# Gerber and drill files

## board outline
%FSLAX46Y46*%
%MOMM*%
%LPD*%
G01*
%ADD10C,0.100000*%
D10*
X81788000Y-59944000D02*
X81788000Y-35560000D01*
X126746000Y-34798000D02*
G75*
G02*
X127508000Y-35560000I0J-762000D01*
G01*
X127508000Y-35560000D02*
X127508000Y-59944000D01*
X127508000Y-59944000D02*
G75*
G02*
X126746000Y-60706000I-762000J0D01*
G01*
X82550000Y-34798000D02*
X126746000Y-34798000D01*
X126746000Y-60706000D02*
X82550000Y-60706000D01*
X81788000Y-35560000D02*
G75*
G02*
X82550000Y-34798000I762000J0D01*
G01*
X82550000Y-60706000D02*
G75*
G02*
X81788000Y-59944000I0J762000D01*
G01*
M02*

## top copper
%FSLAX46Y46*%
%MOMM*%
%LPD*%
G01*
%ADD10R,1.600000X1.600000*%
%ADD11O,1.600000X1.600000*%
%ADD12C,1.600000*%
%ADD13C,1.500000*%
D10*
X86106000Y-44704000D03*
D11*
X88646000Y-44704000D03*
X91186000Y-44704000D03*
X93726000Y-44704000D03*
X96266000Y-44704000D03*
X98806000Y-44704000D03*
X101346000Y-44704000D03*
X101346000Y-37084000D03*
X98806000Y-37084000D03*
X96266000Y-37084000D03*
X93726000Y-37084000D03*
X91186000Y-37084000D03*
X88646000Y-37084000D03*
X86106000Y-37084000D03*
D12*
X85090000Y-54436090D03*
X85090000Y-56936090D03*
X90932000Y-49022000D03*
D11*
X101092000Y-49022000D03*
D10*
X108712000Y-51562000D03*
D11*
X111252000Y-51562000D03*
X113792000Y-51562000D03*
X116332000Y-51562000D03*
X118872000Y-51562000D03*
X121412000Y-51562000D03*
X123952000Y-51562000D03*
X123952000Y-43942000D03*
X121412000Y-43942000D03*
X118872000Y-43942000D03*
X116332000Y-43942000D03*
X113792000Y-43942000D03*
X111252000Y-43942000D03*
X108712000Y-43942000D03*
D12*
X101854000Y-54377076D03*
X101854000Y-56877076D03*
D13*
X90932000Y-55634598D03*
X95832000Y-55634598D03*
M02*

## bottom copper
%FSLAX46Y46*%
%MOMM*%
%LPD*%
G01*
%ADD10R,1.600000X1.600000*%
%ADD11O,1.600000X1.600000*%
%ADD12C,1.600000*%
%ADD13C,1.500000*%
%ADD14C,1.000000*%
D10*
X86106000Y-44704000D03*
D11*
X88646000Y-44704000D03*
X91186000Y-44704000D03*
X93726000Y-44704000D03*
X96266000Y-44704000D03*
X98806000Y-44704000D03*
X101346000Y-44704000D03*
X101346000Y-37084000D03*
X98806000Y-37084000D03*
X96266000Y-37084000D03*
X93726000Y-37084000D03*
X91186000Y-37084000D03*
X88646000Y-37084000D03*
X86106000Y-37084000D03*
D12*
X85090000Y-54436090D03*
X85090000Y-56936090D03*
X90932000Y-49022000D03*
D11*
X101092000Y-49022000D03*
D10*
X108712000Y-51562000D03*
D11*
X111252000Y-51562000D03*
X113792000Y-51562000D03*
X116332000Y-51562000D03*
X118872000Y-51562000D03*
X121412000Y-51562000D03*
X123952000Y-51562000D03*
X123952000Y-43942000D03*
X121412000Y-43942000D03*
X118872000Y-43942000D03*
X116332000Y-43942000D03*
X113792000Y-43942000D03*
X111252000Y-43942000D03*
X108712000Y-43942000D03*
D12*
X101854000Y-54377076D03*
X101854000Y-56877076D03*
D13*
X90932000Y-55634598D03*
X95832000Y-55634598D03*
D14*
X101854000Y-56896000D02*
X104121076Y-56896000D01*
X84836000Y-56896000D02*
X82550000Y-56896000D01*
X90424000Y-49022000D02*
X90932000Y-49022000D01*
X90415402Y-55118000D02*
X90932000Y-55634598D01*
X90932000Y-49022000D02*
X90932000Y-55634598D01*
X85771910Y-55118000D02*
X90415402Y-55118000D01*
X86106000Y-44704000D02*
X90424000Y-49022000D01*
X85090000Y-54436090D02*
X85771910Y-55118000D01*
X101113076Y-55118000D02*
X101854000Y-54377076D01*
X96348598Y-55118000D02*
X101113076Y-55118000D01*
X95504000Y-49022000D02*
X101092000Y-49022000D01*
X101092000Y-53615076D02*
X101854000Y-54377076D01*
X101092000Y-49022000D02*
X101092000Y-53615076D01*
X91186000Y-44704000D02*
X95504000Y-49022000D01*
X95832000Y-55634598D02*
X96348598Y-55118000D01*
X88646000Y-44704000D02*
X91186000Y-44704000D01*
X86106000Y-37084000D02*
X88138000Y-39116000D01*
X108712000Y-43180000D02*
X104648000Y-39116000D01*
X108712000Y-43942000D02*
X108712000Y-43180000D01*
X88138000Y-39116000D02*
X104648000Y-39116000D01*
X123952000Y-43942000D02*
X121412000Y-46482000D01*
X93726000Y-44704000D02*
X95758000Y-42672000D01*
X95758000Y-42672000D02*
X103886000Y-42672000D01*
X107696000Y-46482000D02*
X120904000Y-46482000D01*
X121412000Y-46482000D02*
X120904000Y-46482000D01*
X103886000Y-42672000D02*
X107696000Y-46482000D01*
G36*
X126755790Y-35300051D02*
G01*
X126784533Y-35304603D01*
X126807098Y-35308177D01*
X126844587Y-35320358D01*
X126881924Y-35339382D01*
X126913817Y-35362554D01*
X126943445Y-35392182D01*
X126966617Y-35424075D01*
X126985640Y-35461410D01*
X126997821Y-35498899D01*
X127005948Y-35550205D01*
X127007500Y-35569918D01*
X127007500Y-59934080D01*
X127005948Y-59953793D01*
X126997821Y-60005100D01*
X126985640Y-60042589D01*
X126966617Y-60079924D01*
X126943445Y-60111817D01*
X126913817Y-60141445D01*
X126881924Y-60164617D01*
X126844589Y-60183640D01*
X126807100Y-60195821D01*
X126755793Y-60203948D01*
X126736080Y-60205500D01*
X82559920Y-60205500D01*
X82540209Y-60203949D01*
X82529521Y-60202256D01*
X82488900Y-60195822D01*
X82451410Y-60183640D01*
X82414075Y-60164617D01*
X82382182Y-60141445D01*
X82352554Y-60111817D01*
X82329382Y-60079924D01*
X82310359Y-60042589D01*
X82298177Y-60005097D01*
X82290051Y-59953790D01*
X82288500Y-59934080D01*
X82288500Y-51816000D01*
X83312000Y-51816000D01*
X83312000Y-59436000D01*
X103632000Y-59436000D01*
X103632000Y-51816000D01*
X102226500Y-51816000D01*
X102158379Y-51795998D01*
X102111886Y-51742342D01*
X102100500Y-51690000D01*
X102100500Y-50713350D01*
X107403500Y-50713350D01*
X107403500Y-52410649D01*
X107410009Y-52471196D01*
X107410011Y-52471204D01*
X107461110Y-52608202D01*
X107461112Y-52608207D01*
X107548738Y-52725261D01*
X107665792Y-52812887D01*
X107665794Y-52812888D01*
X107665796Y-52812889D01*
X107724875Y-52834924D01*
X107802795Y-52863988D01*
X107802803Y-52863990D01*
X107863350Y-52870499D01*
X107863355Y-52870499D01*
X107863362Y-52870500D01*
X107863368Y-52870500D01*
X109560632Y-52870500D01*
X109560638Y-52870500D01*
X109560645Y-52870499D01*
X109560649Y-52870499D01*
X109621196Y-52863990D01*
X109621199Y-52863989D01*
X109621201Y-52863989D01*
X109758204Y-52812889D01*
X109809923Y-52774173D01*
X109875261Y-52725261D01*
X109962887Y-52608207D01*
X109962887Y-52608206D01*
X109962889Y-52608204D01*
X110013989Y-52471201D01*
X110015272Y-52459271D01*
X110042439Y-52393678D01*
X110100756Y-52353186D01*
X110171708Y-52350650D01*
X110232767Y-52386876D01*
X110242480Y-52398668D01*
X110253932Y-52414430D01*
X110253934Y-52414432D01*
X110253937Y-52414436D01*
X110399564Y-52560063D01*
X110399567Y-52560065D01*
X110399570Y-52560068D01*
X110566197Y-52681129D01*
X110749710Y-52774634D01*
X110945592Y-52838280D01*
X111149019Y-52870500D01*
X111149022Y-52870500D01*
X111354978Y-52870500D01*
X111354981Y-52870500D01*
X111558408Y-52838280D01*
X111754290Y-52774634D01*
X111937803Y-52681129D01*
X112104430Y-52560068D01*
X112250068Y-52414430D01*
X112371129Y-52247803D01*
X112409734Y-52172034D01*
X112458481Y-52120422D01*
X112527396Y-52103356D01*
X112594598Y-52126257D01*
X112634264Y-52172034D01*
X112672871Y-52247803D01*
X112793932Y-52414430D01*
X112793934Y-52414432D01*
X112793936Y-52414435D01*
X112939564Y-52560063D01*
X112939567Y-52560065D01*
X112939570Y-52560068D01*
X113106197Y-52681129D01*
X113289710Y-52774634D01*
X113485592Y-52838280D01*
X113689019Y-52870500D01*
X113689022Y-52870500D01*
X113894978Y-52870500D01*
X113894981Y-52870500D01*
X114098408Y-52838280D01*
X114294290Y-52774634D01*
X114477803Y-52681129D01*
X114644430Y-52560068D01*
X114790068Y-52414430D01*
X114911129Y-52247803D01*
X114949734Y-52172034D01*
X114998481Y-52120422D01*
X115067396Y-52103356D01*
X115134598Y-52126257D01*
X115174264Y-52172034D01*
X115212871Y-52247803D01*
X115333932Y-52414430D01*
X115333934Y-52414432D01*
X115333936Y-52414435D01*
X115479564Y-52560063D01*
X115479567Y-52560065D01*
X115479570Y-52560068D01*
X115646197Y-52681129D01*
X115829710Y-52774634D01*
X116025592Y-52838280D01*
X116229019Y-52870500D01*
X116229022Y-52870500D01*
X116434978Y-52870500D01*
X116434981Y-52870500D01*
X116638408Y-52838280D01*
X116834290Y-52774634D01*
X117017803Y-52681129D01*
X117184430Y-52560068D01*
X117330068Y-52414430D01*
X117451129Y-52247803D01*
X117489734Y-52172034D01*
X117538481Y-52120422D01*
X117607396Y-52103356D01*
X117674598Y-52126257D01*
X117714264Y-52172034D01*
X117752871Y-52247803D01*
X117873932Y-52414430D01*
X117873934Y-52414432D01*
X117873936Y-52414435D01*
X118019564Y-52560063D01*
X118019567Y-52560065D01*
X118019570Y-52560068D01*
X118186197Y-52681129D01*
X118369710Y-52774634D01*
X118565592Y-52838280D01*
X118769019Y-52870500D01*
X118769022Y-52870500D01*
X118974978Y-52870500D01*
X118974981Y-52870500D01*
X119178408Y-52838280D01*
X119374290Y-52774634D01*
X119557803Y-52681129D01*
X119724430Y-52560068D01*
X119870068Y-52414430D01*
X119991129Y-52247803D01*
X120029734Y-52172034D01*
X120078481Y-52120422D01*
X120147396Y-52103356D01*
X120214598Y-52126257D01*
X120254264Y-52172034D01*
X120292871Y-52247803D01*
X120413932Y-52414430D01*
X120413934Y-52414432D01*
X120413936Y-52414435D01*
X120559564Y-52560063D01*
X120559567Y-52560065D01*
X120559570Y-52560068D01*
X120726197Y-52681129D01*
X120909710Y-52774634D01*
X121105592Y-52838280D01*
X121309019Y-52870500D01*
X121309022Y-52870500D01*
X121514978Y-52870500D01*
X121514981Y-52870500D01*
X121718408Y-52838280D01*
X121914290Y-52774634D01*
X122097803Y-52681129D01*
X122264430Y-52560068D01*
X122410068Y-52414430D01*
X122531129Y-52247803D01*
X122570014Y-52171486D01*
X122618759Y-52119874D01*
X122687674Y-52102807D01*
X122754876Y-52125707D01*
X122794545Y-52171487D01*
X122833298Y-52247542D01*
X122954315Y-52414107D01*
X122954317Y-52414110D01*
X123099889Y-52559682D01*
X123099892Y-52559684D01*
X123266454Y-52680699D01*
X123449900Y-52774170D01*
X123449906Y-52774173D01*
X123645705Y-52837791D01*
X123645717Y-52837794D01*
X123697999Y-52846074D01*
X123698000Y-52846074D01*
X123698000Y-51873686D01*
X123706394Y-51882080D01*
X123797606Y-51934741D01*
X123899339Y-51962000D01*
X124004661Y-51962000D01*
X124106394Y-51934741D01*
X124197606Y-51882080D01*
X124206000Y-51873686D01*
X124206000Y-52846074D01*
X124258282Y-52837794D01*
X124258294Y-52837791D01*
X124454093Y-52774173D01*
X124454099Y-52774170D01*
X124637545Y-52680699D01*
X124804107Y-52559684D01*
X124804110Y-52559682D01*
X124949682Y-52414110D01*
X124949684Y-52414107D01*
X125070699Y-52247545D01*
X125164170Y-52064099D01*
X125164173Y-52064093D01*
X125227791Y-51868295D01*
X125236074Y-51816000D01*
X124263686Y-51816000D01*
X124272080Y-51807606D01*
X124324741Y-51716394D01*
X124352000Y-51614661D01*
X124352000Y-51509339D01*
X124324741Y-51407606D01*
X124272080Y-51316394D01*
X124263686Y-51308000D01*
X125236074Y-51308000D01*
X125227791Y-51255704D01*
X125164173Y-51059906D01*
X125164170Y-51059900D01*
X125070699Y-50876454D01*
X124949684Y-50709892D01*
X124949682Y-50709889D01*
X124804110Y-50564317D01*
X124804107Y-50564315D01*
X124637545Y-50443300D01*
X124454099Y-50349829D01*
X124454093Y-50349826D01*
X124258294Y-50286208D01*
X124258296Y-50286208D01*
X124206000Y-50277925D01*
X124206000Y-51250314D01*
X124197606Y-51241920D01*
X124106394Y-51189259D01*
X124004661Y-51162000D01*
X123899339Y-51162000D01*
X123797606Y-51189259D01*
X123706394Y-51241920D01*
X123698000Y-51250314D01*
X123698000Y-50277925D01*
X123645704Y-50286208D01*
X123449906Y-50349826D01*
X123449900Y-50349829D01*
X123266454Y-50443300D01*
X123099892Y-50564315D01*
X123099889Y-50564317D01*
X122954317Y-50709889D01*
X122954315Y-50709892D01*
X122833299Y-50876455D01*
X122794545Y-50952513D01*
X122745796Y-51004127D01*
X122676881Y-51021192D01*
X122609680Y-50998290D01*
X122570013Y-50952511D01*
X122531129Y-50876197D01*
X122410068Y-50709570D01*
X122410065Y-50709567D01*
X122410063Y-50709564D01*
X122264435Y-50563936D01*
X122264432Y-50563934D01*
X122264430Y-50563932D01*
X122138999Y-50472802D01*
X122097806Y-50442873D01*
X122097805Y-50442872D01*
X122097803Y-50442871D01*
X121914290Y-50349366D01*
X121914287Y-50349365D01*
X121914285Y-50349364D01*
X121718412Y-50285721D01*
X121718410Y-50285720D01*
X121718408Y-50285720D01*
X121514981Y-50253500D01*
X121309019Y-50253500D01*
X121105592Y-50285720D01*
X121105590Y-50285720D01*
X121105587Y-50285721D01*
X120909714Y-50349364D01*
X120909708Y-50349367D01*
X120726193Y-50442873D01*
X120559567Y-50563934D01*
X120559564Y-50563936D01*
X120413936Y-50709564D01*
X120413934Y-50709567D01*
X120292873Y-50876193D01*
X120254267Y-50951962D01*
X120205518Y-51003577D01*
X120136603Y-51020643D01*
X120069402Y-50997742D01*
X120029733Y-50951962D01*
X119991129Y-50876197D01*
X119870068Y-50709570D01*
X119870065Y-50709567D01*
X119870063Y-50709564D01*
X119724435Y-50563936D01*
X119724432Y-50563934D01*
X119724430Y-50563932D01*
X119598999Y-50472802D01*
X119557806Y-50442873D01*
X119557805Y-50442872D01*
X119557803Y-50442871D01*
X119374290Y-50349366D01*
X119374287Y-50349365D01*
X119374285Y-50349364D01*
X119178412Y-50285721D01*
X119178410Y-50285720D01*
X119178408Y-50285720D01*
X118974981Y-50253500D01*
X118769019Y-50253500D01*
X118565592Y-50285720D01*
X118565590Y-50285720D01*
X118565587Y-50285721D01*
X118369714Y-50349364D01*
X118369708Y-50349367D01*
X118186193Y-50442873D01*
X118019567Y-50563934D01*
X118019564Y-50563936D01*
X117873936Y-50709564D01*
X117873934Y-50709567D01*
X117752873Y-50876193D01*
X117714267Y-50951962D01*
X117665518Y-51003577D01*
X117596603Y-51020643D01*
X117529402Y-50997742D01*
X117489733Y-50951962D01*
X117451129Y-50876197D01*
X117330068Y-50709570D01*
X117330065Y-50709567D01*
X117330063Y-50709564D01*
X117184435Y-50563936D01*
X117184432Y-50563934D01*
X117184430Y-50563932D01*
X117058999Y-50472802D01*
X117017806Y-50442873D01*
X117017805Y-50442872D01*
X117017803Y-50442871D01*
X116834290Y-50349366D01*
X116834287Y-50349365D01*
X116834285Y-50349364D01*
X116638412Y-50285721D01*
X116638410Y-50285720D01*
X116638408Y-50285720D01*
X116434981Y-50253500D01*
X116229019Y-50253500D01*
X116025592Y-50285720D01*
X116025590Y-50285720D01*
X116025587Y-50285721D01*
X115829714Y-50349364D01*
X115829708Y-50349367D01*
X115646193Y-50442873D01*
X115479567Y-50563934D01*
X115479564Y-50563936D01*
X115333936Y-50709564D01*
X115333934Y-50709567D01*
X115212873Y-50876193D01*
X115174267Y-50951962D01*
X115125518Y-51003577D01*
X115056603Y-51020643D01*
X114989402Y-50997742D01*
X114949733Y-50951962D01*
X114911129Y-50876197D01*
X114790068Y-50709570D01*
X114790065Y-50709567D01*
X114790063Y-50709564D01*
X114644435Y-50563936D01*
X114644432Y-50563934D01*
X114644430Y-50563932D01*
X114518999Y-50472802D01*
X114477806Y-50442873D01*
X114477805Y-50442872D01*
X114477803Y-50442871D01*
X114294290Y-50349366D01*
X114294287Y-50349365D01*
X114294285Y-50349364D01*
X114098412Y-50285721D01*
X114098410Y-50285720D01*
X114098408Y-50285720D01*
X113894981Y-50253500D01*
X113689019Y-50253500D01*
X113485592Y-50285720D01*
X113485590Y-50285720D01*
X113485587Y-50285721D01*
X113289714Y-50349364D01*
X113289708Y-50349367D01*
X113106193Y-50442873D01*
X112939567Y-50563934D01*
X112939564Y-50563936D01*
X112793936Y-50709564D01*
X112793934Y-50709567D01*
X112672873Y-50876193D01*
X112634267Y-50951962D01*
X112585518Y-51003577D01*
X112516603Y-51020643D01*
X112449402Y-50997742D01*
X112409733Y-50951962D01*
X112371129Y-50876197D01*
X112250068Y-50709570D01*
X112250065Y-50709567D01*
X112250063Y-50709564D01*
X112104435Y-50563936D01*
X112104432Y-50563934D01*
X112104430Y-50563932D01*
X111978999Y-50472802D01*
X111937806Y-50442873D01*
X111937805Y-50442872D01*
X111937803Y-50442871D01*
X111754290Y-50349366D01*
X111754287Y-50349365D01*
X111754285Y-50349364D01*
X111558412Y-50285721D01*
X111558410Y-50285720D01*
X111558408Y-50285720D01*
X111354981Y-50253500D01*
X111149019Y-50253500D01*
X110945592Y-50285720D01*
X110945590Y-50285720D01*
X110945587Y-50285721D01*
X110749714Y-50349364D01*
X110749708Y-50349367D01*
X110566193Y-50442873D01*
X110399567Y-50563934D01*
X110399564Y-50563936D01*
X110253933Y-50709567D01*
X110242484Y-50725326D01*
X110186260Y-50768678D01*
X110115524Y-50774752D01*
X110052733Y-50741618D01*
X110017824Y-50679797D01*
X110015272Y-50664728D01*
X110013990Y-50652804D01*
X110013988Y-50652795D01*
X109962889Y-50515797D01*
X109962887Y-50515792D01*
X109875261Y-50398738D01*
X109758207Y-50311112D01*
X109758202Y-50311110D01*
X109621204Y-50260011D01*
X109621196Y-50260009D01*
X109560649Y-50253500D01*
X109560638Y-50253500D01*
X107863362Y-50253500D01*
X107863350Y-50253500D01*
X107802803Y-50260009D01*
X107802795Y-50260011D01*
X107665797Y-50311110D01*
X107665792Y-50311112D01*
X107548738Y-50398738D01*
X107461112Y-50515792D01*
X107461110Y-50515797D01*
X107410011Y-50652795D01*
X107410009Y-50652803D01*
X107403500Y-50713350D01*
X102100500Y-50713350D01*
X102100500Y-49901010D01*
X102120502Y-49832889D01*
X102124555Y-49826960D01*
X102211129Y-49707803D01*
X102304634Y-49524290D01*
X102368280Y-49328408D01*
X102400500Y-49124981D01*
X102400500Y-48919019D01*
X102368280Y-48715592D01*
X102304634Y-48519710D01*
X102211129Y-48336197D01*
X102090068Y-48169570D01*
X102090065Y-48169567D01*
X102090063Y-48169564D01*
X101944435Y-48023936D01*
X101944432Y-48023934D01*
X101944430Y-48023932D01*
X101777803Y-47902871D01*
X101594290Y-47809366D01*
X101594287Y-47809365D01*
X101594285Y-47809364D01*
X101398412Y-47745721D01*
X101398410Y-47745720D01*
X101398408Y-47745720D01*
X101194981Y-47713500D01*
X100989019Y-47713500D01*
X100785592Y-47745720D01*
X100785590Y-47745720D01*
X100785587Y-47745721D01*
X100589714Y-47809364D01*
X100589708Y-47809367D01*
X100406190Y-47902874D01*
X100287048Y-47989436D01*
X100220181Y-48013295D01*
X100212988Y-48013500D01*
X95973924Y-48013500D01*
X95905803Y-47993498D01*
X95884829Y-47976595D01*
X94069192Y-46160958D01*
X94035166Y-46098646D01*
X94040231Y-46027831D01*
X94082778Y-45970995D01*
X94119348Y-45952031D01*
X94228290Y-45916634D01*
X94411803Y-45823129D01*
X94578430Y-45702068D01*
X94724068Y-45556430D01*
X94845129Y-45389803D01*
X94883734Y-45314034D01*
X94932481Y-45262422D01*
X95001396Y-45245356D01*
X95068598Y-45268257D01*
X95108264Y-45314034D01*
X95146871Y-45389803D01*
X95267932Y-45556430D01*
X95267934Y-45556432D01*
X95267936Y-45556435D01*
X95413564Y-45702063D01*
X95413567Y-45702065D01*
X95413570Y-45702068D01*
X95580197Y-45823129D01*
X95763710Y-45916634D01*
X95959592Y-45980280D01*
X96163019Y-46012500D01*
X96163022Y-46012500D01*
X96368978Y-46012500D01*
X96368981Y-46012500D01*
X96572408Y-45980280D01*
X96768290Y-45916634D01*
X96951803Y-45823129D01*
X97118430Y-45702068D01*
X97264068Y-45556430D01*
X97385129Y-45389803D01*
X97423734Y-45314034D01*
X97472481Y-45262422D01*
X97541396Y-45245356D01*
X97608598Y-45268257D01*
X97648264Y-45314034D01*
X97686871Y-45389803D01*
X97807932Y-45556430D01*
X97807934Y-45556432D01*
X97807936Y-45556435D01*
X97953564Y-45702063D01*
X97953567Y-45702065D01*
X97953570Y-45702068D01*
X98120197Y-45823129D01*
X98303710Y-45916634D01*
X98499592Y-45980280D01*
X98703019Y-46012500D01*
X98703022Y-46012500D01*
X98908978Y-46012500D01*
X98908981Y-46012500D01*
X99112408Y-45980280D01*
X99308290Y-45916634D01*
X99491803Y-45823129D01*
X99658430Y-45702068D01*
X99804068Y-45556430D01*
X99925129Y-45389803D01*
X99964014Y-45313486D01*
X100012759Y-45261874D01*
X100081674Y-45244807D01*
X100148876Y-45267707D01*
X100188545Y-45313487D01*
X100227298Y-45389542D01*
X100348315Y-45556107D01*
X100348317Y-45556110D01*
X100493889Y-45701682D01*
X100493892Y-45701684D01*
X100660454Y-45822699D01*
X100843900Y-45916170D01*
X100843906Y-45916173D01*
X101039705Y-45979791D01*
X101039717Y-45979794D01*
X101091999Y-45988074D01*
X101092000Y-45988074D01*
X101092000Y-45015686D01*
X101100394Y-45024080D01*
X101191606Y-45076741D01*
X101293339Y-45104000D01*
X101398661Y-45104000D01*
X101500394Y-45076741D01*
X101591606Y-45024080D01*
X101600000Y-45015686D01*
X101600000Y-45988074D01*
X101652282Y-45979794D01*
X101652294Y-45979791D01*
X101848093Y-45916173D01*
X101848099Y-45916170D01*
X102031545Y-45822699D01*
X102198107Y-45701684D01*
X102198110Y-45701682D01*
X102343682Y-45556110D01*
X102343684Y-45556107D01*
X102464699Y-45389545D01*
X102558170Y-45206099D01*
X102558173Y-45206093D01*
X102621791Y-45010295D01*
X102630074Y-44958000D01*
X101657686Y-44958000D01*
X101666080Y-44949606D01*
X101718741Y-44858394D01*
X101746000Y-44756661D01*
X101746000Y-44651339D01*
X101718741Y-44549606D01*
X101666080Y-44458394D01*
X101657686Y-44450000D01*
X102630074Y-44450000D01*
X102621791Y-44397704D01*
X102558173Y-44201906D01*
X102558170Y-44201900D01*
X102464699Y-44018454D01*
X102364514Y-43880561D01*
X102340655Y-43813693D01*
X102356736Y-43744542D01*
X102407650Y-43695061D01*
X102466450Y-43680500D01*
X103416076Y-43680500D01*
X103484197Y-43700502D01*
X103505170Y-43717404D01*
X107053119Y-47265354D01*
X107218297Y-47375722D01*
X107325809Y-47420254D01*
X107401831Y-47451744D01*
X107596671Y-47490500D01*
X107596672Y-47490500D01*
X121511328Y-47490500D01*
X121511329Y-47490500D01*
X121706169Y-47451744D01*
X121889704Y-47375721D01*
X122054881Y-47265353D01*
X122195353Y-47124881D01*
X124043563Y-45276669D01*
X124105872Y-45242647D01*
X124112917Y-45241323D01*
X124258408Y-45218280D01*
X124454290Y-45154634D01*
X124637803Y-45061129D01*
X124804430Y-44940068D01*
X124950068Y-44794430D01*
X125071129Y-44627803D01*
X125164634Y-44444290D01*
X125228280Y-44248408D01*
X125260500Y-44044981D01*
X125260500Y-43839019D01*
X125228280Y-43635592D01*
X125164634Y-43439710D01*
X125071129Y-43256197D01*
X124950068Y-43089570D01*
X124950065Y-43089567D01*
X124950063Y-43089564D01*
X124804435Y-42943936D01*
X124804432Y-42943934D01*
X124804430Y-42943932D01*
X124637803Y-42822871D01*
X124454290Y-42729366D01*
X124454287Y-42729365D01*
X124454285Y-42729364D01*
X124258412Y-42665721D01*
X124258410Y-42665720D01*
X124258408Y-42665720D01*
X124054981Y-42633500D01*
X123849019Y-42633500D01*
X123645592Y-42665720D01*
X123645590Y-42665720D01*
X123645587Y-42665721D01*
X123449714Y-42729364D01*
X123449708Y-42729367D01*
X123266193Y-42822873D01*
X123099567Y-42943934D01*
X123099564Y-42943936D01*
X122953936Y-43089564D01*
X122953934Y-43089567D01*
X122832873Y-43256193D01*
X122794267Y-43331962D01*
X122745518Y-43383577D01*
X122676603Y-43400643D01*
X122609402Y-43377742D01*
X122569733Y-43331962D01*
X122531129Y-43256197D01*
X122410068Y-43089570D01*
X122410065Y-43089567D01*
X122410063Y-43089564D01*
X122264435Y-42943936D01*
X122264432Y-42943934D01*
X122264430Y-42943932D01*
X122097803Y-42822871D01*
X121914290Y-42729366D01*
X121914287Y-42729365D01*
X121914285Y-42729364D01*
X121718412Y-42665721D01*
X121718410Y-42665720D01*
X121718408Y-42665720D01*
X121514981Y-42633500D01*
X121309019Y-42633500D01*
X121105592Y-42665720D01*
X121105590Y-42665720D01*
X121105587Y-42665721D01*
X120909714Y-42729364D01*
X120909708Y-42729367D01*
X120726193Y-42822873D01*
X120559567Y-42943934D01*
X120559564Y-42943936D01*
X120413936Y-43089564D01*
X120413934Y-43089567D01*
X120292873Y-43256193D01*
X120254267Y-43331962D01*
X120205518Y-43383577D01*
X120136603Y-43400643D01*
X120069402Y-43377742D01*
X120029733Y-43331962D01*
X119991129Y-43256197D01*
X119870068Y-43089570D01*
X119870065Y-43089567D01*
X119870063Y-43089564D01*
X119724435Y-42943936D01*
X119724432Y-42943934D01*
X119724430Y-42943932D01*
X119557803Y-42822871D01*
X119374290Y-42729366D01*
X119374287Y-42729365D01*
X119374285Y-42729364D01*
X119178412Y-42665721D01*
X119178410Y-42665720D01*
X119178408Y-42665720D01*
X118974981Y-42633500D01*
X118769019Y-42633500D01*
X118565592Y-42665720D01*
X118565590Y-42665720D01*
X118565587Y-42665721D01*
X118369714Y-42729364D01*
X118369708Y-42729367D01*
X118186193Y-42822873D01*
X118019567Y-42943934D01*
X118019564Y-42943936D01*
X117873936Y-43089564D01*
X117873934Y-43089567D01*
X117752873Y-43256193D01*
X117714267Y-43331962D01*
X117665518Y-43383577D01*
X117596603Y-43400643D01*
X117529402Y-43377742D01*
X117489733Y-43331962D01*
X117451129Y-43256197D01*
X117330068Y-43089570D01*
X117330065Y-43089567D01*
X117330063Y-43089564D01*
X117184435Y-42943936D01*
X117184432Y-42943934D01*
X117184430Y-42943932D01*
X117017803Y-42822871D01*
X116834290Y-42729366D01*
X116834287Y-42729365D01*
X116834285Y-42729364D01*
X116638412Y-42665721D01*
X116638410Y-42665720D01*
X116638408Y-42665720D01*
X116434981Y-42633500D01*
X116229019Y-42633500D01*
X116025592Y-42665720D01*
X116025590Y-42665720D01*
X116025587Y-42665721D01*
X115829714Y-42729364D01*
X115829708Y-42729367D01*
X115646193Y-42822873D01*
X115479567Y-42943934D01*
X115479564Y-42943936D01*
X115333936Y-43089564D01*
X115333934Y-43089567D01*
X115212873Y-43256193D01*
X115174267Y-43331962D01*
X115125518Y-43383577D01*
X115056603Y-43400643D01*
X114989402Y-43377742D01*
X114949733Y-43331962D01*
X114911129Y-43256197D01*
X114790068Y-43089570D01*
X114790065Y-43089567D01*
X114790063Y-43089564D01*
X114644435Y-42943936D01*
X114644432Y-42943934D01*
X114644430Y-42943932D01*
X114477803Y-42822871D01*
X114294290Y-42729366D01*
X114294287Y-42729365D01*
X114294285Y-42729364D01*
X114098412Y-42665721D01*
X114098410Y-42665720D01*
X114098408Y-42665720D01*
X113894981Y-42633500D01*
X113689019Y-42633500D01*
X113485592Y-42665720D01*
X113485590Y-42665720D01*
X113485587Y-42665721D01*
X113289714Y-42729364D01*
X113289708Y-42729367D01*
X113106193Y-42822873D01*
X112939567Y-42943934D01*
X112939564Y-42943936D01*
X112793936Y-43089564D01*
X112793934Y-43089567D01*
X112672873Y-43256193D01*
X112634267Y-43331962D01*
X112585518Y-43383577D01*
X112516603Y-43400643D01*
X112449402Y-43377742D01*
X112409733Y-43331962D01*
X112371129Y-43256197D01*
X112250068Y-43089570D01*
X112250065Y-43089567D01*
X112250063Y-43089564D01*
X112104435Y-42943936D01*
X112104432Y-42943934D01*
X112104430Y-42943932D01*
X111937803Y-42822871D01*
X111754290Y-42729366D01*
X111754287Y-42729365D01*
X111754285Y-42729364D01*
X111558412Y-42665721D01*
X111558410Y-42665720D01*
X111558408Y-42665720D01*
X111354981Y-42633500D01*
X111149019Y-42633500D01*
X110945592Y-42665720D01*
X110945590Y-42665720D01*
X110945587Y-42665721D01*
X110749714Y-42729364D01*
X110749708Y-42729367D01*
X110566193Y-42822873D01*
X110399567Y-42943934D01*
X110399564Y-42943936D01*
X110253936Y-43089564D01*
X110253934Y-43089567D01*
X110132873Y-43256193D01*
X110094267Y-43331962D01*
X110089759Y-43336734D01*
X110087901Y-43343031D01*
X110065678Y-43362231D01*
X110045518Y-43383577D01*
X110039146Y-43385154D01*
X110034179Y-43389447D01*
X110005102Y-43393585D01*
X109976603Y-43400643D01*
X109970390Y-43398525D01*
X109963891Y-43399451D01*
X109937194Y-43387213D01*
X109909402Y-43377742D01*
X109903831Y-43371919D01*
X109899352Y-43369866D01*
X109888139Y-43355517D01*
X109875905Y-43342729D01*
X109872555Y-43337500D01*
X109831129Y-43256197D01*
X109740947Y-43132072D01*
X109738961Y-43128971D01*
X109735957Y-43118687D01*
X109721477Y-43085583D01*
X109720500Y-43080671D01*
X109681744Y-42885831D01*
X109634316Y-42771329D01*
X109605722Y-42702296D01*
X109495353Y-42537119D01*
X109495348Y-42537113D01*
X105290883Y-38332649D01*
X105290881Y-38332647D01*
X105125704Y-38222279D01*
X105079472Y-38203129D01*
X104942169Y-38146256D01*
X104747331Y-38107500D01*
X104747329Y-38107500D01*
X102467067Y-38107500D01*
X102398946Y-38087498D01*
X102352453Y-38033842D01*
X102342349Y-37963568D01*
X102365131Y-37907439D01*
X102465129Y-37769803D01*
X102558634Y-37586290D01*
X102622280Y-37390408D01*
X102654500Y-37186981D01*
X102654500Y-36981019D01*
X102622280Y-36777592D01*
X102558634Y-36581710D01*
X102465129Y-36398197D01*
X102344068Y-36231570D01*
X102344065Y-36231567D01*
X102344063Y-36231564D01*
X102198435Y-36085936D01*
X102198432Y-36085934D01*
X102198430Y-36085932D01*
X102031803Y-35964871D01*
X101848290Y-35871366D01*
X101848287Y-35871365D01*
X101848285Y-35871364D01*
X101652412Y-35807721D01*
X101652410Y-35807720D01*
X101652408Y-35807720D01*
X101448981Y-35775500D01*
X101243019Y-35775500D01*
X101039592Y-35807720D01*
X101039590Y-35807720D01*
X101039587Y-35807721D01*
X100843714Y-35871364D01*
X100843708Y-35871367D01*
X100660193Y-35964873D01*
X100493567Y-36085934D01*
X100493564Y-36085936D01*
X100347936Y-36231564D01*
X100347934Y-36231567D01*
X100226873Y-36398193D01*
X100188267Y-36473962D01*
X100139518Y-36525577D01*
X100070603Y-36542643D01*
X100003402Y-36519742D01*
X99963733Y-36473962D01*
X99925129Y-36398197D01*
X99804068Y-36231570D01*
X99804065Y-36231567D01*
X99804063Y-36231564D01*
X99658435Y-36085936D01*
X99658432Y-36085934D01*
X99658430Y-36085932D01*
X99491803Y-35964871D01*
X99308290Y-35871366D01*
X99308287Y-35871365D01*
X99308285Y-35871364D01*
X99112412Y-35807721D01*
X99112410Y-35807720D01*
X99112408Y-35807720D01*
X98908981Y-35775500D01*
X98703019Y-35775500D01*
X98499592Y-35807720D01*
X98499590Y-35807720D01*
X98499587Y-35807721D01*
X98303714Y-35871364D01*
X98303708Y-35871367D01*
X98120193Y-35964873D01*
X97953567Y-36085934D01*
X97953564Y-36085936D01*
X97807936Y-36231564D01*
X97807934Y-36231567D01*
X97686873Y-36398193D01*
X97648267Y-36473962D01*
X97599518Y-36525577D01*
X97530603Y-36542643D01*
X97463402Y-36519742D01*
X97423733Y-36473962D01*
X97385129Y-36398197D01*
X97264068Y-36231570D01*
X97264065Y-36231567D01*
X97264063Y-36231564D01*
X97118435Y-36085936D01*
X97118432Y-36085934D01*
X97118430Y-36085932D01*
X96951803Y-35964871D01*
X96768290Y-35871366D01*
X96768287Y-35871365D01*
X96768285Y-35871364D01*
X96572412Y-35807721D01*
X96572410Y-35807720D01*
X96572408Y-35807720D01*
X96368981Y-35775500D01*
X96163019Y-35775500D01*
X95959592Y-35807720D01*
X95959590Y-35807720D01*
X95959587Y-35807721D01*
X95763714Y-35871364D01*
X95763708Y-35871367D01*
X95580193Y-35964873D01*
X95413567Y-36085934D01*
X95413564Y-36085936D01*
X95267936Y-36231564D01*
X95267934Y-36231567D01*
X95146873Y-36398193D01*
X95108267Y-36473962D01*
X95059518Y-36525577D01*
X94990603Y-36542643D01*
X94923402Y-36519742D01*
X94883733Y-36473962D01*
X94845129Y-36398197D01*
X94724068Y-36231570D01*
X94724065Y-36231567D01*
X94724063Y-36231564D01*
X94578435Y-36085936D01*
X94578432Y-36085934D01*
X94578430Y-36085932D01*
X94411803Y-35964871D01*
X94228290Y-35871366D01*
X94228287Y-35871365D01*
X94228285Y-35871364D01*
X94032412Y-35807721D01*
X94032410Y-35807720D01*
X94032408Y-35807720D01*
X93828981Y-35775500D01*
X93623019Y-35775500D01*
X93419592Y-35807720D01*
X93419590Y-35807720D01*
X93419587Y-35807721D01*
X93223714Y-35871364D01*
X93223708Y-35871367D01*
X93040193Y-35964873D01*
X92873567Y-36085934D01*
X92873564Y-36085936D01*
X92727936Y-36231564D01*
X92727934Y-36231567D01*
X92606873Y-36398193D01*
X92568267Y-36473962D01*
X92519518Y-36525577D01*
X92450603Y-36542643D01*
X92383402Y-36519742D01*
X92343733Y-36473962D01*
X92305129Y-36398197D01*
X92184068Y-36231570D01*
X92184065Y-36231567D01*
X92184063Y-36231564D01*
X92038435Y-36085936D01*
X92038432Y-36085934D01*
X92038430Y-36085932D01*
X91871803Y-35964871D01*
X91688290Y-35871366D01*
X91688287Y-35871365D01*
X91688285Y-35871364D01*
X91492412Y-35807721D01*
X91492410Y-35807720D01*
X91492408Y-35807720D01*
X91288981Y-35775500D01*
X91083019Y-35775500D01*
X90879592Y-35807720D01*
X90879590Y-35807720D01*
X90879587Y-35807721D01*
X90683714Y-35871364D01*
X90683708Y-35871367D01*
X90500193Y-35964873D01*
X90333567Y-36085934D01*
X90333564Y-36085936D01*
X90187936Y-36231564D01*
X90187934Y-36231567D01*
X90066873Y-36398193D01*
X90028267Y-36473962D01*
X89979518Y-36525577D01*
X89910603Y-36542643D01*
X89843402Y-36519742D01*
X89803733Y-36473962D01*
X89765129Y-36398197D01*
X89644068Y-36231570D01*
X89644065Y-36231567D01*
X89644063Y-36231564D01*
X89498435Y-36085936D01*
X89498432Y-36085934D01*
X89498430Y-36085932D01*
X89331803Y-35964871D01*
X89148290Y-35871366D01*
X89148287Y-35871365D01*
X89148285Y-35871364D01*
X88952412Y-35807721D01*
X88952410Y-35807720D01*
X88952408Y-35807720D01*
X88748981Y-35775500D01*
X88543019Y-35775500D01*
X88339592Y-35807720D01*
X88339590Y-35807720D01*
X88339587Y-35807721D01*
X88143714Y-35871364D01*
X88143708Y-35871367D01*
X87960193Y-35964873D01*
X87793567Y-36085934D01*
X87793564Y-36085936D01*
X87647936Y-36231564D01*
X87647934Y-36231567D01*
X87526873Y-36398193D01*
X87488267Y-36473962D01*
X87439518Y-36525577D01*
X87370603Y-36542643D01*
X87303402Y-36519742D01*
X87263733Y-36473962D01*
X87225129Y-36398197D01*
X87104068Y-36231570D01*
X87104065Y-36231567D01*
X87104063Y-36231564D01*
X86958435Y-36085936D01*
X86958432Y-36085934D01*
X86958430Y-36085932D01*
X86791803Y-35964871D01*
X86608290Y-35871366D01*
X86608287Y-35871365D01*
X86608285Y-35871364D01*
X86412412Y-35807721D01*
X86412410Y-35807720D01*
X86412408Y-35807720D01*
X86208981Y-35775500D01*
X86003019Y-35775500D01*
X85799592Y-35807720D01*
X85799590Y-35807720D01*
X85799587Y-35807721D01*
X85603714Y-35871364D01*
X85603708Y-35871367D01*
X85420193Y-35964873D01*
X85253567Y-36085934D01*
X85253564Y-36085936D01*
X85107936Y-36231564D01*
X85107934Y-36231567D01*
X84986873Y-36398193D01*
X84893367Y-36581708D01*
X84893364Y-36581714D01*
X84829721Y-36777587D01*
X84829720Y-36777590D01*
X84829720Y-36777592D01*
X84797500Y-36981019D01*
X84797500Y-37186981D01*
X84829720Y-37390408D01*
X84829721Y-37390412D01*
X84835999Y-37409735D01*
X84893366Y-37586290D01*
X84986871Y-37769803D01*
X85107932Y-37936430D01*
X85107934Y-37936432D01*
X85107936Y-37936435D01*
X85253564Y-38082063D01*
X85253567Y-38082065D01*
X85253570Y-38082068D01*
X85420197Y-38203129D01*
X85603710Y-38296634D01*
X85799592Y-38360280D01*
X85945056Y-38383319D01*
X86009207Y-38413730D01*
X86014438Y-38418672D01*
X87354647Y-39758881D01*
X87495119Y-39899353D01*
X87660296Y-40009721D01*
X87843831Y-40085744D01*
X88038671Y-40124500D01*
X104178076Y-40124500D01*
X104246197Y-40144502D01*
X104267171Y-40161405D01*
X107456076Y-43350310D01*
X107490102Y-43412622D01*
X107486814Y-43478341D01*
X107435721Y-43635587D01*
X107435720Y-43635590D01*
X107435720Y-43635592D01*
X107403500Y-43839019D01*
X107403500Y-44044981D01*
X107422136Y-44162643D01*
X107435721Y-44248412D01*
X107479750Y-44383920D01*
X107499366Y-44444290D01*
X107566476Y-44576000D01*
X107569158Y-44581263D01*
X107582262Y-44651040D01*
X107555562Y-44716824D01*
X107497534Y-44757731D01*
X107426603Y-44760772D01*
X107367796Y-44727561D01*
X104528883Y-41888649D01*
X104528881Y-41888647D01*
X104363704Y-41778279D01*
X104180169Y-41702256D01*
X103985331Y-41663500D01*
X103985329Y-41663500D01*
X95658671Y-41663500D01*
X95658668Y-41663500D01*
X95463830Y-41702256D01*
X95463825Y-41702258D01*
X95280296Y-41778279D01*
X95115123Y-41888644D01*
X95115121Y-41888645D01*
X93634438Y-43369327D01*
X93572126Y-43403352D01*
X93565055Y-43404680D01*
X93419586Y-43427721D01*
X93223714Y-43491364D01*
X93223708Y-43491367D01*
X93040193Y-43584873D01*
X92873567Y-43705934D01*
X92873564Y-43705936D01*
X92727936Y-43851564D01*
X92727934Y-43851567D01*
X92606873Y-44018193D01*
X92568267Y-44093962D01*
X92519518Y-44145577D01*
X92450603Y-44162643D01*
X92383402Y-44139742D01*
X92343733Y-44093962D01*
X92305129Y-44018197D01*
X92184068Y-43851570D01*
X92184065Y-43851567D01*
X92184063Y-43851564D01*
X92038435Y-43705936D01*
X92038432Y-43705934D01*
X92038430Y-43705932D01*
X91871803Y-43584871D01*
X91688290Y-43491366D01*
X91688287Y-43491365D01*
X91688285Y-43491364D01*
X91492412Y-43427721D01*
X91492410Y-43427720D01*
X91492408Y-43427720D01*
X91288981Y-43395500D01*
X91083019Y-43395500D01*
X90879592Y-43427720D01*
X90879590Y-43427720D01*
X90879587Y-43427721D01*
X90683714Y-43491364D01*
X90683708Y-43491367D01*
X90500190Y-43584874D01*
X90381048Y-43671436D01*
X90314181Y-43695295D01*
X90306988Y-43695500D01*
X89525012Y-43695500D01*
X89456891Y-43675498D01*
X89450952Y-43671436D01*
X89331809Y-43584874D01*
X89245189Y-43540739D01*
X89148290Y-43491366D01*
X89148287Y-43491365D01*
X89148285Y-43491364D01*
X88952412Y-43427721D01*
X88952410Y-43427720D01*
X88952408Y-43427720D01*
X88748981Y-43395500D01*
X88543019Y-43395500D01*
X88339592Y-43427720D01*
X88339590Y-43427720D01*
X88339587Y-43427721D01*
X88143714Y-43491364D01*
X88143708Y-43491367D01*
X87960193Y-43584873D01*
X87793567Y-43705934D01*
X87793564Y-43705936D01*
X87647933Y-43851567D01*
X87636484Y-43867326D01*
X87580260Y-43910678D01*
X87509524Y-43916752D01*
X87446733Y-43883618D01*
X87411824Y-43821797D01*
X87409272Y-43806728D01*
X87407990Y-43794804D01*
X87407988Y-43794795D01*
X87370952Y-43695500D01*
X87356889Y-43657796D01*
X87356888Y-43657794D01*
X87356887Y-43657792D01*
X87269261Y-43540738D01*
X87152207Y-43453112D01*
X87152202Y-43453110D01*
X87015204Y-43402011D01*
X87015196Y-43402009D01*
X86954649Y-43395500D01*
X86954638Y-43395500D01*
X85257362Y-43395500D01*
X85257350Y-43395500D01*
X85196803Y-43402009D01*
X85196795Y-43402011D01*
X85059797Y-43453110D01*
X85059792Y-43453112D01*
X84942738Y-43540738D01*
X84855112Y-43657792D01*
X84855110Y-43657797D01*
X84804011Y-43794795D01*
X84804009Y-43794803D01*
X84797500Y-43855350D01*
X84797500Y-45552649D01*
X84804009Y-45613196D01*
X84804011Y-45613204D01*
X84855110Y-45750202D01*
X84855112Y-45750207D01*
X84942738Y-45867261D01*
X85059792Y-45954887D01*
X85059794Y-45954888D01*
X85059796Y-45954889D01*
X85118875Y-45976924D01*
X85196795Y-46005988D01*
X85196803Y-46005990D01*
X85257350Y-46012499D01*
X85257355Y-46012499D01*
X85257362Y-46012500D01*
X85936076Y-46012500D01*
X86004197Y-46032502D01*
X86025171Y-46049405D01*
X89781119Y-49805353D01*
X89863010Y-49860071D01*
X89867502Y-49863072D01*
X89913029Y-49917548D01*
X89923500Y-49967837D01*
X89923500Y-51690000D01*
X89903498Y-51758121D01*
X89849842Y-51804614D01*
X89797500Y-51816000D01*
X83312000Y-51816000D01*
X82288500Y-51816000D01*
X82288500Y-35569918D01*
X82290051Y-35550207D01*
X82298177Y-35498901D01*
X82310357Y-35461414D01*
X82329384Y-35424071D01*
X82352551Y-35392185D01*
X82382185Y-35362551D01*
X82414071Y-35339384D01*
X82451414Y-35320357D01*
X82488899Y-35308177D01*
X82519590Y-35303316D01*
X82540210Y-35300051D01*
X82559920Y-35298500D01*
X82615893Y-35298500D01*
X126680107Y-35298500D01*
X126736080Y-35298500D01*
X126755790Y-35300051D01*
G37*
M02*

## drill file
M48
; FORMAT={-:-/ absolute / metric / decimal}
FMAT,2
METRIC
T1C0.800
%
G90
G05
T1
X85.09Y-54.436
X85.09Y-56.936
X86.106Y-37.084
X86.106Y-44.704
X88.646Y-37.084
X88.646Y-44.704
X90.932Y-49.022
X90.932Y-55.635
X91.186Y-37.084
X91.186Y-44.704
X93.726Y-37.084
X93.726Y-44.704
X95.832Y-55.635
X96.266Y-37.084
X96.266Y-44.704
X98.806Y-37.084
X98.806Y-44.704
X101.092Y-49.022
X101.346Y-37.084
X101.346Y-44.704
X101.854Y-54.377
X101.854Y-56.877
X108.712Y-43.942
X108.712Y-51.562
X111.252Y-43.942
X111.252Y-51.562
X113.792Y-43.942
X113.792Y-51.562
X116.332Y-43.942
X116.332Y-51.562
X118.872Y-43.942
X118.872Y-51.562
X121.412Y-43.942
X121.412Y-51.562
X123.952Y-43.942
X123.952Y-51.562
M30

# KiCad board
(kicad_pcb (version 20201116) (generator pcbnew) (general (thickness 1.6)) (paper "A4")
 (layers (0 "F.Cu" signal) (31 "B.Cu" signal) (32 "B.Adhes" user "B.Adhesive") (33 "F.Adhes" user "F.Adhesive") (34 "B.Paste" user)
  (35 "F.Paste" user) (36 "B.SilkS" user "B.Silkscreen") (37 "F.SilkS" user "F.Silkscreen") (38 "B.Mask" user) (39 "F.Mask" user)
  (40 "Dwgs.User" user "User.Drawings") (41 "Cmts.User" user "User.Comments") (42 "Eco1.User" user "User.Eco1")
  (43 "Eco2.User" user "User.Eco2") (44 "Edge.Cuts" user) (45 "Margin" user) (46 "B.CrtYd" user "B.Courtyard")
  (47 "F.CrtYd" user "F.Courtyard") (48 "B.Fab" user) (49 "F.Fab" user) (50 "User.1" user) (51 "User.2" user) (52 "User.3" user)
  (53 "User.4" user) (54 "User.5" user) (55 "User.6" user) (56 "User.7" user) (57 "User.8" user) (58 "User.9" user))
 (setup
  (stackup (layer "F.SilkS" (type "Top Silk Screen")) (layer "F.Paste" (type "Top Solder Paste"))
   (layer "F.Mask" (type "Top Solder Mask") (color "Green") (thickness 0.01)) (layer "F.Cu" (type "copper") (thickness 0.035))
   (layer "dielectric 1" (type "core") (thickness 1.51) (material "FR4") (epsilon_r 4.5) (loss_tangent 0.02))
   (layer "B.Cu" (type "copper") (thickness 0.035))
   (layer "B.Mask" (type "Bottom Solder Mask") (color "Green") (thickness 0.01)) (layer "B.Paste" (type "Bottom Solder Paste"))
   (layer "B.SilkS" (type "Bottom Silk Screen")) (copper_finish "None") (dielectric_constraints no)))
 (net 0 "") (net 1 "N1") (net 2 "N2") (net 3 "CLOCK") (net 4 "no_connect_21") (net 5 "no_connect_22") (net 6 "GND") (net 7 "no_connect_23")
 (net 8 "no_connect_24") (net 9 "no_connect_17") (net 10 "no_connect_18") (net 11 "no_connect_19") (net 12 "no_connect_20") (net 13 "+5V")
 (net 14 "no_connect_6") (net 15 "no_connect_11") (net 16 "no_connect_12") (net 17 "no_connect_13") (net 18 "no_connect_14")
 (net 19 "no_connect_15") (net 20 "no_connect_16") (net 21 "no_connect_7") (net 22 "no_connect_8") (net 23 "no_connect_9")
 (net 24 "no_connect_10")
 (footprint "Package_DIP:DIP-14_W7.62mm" (layer "F.Cu") (at 86.106 44.704 90)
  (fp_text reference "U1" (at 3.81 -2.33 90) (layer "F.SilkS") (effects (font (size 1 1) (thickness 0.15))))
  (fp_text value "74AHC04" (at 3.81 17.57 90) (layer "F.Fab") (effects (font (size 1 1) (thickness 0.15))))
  (pad "1" thru_hole rect (at 0 0 90) (size 1.6 1.6) (drill 0.8) (layers *.Cu *.Mask) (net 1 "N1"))
  (pad "2" thru_hole oval (at 0 2.54 90) (size 1.6 1.6) (drill 0.8) (layers *.Cu *.Mask) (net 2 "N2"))
  (pad "3" thru_hole oval (at 0 5.08 90) (size 1.6 1.6) (drill 0.8) (layers *.Cu *.Mask) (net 2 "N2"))
  (pad "4" thru_hole oval (at 0 7.62 90) (size 1.6 1.6) (drill 0.8) (layers *.Cu *.Mask) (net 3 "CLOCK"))
  (pad "5" thru_hole oval (at 0 10.16 90) (size 1.6 1.6) (drill 0.8) (layers *.Cu *.Mask) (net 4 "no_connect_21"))
  (pad "6" thru_hole oval (at 0 12.7 90) (size 1.6 1.6) (drill 0.8) (layers *.Cu *.Mask) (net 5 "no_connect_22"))
  (pad "7" thru_hole oval (at 0 15.24 90) (size 1.6 1.6) (drill 0.8) (layers *.Cu *.Mask) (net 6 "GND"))
  (pad "8" thru_hole oval (at 7.62 15.24 90) (size 1.6 1.6) (drill 0.8) (layers *.Cu *.Mask) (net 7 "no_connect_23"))
  (pad "9" thru_hole oval (at 7.62 12.7 90) (size 1.6 1.6) (drill 0.8) (layers *.Cu *.Mask) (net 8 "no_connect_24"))
  (pad "10" thru_hole oval (at 7.62 10.16 90) (size 1.6 1.6) (drill 0.8) (layers *.Cu *.Mask) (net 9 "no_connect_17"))
  (pad "11" thru_hole oval (at 7.62 7.62 90) (size 1.6 1.6) (drill 0.8) (layers *.Cu *.Mask) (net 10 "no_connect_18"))
  (pad "12" thru_hole oval (at 7.62 5.08 90) (size 1.6 1.6) (drill 0.8) (layers *.Cu *.Mask) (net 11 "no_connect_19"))
  (pad "13" thru_hole oval (at 7.62 2.54 90) (size 1.6 1.6) (drill 0.8) (layers *.Cu *.Mask) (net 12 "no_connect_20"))
  (pad "14" thru_hole oval (at 7.62 0 90) (size 1.6 1.6) (drill 0.8) (layers *.Cu *.Mask) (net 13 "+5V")))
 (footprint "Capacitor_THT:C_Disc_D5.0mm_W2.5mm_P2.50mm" (layer "F.Cu") (at 85.09 54.43609 -90)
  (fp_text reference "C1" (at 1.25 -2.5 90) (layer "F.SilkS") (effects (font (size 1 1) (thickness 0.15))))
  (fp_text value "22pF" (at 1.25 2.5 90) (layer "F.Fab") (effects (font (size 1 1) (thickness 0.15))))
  (pad "1" thru_hole circle (at 0 0 270) (size 1.6 1.6) (drill 0.8) (layers *.Cu *.Mask) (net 1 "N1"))
  (pad "2" thru_hole circle (at 2.5 0 270) (size 1.6 1.6) (drill 0.8) (layers *.Cu *.Mask) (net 6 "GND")))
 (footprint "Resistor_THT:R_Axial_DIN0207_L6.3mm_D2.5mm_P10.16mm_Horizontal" (layer "F.Cu") (at 90.932 49.022)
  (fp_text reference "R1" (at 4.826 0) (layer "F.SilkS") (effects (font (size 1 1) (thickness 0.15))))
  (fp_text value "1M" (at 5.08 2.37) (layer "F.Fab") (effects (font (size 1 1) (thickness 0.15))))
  (pad "1" thru_hole circle (at 0 0) (size 1.6 1.6) (drill 0.8) (layers *.Cu *.Mask) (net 1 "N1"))
  (pad "2" thru_hole oval (at 10.16 0) (size 1.6 1.6) (drill 0.8) (layers *.Cu *.Mask) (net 2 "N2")))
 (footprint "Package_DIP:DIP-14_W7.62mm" (layer "F.Cu") (at 108.712 51.562 90)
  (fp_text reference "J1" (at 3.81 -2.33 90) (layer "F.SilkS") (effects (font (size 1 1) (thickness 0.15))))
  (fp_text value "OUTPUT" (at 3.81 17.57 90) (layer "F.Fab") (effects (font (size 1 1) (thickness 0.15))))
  (pad "1" thru_hole rect (at 0 0 90) (size 1.6 1.6) (drill 0.8) (layers *.Cu *.Mask) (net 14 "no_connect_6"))
  (pad "2" thru_hole oval (at 0 2.54 90) (size 1.6 1.6) (drill 0.8) (layers *.Cu *.Mask) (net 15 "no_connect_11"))
  (pad "3" thru_hole oval (at 0 5.08 90) (size 1.6 1.6) (drill 0.8) (layers *.Cu *.Mask) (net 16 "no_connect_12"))
  (pad "4" thru_hole oval (at 0 7.62 90) (size 1.6 1.6) (drill 0.8) (layers *.Cu *.Mask) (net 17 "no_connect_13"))
  (pad "5" thru_hole oval (at 0 10.16 90) (size 1.6 1.6) (drill 0.8) (layers *.Cu *.Mask) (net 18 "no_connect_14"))
  (pad "6" thru_hole oval (at 0 12.7 90) (size 1.6 1.6) (drill 0.8) (layers *.Cu *.Mask) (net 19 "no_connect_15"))
  (pad "7" thru_hole oval (at 0 15.24 90) (size 1.6 1.6) (drill 0.8) (layers *.Cu *.Mask) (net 6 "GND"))
  (pad "8" thru_hole oval (at 7.62 15.24 90) (size 1.6 1.6) (drill 0.8) (layers *.Cu *.Mask) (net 3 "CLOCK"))
  (pad "9" thru_hole oval (at 7.62 12.7 90) (size 1.6 1.6) (drill 0.8) (layers *.Cu *.Mask) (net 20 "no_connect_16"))
  (pad "10" thru_hole oval (at 7.62 10.16 90) (size 1.6 1.6) (drill 0.8) (layers *.Cu *.Mask) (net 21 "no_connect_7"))
  (pad "11" thru_hole oval (at 7.62 7.62 90) (size 1.6 1.6) (drill 0.8) (layers *.Cu *.Mask) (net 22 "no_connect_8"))
  (pad "12" thru_hole oval (at 7.62 5.08 90) (size 1.6 1.6) (drill 0.8) (layers *.Cu *.Mask) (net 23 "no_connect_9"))
  (pad "13" thru_hole oval (at 7.62 2.54 90) (size 1.6 1.6) (drill 0.8) (layers *.Cu *.Mask) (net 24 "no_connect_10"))
  (pad "14" thru_hole oval (at 7.62 0 90) (size 1.6 1.6) (drill 0.8) (layers *.Cu *.Mask) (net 13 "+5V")))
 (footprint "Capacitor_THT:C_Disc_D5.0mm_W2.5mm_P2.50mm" (layer "F.Cu") (at 101.854 54.377076 -90)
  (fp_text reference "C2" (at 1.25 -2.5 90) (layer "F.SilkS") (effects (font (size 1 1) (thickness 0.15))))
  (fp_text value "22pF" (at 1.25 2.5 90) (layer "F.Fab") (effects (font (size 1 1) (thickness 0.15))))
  (pad "1" thru_hole circle (at 0 0 270) (size 1.6 1.6) (drill 0.8) (layers *.Cu *.Mask) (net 2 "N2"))
  (pad "2" thru_hole circle (at 2.5 0 270) (size 1.6 1.6) (drill 0.8) (layers *.Cu *.Mask) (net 6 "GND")))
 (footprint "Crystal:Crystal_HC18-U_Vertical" (layer "F.Cu") (at 90.932 55.634598)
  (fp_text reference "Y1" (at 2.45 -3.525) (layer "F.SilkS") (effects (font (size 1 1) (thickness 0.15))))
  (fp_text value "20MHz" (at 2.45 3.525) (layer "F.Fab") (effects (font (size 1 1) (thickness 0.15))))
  (pad "1" thru_hole circle (at 0 0) (size 1.5 1.5) (drill 0.8) (layers *.Cu *.Mask) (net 1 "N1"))
  (pad "2" thru_hole circle (at 4.9 0) (size 1.5 1.5) (drill 0.8) (layers *.Cu *.Mask) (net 2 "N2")))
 (gr_line (start 81.788 59.944) (end 81.788 35.56) (layer "Edge.Cuts") (width 0.1))
 (gr_arc (start 126.746 35.56) (end 127.508 35.56) (angle -90) (layer "Edge.Cuts") (width 0.1))
 (gr_line (start 127.508 35.56) (end 127.508 59.944) (layer "Edge.Cuts") (width 0.1))
 (gr_arc (start 126.746 59.944) (end 126.746 60.706) (angle -90) (layer "Edge.Cuts") (width 0.1))
 (gr_line (start 82.55 34.798) (end 126.746 34.798) (layer "Edge.Cuts") (width 0.1))
 (gr_line (start 126.746 60.706) (end 82.55 60.706) (layer "Edge.Cuts") (width 0.1))
 (gr_arc (start 82.55 35.56) (end 82.55 34.798) (angle -90) (layer "Edge.Cuts") (width 0.1))
 (gr_arc (start 82.55 59.944) (end 81.788 59.944) (angle -90) (layer "Edge.Cuts") (width 0.1))
 (segment (start 101.854 56.896) (end 104.121076 56.896) (width 1) (layer "B.Cu") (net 6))
 (segment (start 84.836 56.896) (end 82.55 56.896) (width 1) (layer "B.Cu") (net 6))
 (segment (start 90.424 49.022) (end 90.932 49.022) (width 1) (layer "B.Cu") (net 1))
 (segment (start 90.415402 55.118) (end 90.932 55.634598) (width 1) (layer "B.Cu") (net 1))
 (segment (start 90.932 49.022) (end 90.932 55.634598) (width 1) (layer "B.Cu") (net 1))
 (segment (start 85.77191 55.118) (end 90.415402 55.118) (width 1) (layer "B.Cu") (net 1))
 (segment (start 86.106 44.704) (end 90.424 49.022) (width 1) (layer "B.Cu") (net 1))
 (segment (start 85.09 54.43609) (end 85.77191 55.118) (width 1) (layer "B.Cu") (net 1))
 (segment (start 101.113076 55.118) (end 101.854 54.377076) (width 1) (layer "B.Cu") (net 2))
 (segment (start 96.348598 55.118) (end 101.113076 55.118) (width 1) (layer "B.Cu") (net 2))
 (segment (start 95.504 49.022) (end 101.092 49.022) (width 1) (layer "B.Cu") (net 2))
 (segment (start 101.092 53.615076) (end 101.854 54.377076) (width 1) (layer "B.Cu") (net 2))
 (segment (start 101.092 49.022) (end 101.092 53.615076) (width 1) (layer "B.Cu") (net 2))
 (segment (start 91.186 44.704) (end 95.504 49.022) (width 1) (layer "B.Cu") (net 2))
 (segment (start 95.832 55.634598) (end 96.348598 55.118) (width 1) (layer "B.Cu") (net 2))
 (segment (start 88.646 44.704) (end 91.186 44.704) (width 1) (layer "B.Cu") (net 2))
 (segment (start 86.106 37.084) (end 88.138 39.116) (width 1) (layer "B.Cu") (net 13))
 (segment (start 108.712 43.18) (end 104.648 39.116) (width 1) (layer "B.Cu") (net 13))
 (segment (start 108.712 43.942) (end 108.712 43.18) (width 1) (layer "B.Cu") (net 13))
 (segment (start 88.138 39.116) (end 104.648 39.116) (width 1) (layer "B.Cu") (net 13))
 (segment (start 123.952 43.942) (end 121.412 46.482) (width 1) (layer "B.Cu") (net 3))
 (segment (start 93.726 44.704) (end 95.758 42.672) (width 1) (layer "B.Cu") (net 3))
 (segment (start 95.758 42.672) (end 103.886 42.672) (width 1) (layer "B.Cu") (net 3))
 (segment (start 107.696 46.482) (end 120.904 46.482) (width 1) (layer "B.Cu") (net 3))
 (segment (start 121.412 46.482) (end 120.904 46.482) (width 1) (layer "B.Cu") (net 3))
 (segment (start 103.886 42.672) (end 107.696 46.482) (width 1) (layer "B.Cu") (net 3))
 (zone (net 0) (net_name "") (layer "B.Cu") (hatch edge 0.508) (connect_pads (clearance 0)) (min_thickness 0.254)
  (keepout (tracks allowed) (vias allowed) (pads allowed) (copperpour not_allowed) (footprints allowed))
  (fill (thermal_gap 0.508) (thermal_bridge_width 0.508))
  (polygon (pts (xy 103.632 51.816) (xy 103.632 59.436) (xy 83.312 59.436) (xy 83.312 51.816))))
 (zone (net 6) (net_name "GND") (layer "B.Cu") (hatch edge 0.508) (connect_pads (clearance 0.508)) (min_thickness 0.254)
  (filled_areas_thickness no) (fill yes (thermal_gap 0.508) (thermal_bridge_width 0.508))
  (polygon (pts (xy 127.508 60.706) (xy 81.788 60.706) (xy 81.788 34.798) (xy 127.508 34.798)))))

